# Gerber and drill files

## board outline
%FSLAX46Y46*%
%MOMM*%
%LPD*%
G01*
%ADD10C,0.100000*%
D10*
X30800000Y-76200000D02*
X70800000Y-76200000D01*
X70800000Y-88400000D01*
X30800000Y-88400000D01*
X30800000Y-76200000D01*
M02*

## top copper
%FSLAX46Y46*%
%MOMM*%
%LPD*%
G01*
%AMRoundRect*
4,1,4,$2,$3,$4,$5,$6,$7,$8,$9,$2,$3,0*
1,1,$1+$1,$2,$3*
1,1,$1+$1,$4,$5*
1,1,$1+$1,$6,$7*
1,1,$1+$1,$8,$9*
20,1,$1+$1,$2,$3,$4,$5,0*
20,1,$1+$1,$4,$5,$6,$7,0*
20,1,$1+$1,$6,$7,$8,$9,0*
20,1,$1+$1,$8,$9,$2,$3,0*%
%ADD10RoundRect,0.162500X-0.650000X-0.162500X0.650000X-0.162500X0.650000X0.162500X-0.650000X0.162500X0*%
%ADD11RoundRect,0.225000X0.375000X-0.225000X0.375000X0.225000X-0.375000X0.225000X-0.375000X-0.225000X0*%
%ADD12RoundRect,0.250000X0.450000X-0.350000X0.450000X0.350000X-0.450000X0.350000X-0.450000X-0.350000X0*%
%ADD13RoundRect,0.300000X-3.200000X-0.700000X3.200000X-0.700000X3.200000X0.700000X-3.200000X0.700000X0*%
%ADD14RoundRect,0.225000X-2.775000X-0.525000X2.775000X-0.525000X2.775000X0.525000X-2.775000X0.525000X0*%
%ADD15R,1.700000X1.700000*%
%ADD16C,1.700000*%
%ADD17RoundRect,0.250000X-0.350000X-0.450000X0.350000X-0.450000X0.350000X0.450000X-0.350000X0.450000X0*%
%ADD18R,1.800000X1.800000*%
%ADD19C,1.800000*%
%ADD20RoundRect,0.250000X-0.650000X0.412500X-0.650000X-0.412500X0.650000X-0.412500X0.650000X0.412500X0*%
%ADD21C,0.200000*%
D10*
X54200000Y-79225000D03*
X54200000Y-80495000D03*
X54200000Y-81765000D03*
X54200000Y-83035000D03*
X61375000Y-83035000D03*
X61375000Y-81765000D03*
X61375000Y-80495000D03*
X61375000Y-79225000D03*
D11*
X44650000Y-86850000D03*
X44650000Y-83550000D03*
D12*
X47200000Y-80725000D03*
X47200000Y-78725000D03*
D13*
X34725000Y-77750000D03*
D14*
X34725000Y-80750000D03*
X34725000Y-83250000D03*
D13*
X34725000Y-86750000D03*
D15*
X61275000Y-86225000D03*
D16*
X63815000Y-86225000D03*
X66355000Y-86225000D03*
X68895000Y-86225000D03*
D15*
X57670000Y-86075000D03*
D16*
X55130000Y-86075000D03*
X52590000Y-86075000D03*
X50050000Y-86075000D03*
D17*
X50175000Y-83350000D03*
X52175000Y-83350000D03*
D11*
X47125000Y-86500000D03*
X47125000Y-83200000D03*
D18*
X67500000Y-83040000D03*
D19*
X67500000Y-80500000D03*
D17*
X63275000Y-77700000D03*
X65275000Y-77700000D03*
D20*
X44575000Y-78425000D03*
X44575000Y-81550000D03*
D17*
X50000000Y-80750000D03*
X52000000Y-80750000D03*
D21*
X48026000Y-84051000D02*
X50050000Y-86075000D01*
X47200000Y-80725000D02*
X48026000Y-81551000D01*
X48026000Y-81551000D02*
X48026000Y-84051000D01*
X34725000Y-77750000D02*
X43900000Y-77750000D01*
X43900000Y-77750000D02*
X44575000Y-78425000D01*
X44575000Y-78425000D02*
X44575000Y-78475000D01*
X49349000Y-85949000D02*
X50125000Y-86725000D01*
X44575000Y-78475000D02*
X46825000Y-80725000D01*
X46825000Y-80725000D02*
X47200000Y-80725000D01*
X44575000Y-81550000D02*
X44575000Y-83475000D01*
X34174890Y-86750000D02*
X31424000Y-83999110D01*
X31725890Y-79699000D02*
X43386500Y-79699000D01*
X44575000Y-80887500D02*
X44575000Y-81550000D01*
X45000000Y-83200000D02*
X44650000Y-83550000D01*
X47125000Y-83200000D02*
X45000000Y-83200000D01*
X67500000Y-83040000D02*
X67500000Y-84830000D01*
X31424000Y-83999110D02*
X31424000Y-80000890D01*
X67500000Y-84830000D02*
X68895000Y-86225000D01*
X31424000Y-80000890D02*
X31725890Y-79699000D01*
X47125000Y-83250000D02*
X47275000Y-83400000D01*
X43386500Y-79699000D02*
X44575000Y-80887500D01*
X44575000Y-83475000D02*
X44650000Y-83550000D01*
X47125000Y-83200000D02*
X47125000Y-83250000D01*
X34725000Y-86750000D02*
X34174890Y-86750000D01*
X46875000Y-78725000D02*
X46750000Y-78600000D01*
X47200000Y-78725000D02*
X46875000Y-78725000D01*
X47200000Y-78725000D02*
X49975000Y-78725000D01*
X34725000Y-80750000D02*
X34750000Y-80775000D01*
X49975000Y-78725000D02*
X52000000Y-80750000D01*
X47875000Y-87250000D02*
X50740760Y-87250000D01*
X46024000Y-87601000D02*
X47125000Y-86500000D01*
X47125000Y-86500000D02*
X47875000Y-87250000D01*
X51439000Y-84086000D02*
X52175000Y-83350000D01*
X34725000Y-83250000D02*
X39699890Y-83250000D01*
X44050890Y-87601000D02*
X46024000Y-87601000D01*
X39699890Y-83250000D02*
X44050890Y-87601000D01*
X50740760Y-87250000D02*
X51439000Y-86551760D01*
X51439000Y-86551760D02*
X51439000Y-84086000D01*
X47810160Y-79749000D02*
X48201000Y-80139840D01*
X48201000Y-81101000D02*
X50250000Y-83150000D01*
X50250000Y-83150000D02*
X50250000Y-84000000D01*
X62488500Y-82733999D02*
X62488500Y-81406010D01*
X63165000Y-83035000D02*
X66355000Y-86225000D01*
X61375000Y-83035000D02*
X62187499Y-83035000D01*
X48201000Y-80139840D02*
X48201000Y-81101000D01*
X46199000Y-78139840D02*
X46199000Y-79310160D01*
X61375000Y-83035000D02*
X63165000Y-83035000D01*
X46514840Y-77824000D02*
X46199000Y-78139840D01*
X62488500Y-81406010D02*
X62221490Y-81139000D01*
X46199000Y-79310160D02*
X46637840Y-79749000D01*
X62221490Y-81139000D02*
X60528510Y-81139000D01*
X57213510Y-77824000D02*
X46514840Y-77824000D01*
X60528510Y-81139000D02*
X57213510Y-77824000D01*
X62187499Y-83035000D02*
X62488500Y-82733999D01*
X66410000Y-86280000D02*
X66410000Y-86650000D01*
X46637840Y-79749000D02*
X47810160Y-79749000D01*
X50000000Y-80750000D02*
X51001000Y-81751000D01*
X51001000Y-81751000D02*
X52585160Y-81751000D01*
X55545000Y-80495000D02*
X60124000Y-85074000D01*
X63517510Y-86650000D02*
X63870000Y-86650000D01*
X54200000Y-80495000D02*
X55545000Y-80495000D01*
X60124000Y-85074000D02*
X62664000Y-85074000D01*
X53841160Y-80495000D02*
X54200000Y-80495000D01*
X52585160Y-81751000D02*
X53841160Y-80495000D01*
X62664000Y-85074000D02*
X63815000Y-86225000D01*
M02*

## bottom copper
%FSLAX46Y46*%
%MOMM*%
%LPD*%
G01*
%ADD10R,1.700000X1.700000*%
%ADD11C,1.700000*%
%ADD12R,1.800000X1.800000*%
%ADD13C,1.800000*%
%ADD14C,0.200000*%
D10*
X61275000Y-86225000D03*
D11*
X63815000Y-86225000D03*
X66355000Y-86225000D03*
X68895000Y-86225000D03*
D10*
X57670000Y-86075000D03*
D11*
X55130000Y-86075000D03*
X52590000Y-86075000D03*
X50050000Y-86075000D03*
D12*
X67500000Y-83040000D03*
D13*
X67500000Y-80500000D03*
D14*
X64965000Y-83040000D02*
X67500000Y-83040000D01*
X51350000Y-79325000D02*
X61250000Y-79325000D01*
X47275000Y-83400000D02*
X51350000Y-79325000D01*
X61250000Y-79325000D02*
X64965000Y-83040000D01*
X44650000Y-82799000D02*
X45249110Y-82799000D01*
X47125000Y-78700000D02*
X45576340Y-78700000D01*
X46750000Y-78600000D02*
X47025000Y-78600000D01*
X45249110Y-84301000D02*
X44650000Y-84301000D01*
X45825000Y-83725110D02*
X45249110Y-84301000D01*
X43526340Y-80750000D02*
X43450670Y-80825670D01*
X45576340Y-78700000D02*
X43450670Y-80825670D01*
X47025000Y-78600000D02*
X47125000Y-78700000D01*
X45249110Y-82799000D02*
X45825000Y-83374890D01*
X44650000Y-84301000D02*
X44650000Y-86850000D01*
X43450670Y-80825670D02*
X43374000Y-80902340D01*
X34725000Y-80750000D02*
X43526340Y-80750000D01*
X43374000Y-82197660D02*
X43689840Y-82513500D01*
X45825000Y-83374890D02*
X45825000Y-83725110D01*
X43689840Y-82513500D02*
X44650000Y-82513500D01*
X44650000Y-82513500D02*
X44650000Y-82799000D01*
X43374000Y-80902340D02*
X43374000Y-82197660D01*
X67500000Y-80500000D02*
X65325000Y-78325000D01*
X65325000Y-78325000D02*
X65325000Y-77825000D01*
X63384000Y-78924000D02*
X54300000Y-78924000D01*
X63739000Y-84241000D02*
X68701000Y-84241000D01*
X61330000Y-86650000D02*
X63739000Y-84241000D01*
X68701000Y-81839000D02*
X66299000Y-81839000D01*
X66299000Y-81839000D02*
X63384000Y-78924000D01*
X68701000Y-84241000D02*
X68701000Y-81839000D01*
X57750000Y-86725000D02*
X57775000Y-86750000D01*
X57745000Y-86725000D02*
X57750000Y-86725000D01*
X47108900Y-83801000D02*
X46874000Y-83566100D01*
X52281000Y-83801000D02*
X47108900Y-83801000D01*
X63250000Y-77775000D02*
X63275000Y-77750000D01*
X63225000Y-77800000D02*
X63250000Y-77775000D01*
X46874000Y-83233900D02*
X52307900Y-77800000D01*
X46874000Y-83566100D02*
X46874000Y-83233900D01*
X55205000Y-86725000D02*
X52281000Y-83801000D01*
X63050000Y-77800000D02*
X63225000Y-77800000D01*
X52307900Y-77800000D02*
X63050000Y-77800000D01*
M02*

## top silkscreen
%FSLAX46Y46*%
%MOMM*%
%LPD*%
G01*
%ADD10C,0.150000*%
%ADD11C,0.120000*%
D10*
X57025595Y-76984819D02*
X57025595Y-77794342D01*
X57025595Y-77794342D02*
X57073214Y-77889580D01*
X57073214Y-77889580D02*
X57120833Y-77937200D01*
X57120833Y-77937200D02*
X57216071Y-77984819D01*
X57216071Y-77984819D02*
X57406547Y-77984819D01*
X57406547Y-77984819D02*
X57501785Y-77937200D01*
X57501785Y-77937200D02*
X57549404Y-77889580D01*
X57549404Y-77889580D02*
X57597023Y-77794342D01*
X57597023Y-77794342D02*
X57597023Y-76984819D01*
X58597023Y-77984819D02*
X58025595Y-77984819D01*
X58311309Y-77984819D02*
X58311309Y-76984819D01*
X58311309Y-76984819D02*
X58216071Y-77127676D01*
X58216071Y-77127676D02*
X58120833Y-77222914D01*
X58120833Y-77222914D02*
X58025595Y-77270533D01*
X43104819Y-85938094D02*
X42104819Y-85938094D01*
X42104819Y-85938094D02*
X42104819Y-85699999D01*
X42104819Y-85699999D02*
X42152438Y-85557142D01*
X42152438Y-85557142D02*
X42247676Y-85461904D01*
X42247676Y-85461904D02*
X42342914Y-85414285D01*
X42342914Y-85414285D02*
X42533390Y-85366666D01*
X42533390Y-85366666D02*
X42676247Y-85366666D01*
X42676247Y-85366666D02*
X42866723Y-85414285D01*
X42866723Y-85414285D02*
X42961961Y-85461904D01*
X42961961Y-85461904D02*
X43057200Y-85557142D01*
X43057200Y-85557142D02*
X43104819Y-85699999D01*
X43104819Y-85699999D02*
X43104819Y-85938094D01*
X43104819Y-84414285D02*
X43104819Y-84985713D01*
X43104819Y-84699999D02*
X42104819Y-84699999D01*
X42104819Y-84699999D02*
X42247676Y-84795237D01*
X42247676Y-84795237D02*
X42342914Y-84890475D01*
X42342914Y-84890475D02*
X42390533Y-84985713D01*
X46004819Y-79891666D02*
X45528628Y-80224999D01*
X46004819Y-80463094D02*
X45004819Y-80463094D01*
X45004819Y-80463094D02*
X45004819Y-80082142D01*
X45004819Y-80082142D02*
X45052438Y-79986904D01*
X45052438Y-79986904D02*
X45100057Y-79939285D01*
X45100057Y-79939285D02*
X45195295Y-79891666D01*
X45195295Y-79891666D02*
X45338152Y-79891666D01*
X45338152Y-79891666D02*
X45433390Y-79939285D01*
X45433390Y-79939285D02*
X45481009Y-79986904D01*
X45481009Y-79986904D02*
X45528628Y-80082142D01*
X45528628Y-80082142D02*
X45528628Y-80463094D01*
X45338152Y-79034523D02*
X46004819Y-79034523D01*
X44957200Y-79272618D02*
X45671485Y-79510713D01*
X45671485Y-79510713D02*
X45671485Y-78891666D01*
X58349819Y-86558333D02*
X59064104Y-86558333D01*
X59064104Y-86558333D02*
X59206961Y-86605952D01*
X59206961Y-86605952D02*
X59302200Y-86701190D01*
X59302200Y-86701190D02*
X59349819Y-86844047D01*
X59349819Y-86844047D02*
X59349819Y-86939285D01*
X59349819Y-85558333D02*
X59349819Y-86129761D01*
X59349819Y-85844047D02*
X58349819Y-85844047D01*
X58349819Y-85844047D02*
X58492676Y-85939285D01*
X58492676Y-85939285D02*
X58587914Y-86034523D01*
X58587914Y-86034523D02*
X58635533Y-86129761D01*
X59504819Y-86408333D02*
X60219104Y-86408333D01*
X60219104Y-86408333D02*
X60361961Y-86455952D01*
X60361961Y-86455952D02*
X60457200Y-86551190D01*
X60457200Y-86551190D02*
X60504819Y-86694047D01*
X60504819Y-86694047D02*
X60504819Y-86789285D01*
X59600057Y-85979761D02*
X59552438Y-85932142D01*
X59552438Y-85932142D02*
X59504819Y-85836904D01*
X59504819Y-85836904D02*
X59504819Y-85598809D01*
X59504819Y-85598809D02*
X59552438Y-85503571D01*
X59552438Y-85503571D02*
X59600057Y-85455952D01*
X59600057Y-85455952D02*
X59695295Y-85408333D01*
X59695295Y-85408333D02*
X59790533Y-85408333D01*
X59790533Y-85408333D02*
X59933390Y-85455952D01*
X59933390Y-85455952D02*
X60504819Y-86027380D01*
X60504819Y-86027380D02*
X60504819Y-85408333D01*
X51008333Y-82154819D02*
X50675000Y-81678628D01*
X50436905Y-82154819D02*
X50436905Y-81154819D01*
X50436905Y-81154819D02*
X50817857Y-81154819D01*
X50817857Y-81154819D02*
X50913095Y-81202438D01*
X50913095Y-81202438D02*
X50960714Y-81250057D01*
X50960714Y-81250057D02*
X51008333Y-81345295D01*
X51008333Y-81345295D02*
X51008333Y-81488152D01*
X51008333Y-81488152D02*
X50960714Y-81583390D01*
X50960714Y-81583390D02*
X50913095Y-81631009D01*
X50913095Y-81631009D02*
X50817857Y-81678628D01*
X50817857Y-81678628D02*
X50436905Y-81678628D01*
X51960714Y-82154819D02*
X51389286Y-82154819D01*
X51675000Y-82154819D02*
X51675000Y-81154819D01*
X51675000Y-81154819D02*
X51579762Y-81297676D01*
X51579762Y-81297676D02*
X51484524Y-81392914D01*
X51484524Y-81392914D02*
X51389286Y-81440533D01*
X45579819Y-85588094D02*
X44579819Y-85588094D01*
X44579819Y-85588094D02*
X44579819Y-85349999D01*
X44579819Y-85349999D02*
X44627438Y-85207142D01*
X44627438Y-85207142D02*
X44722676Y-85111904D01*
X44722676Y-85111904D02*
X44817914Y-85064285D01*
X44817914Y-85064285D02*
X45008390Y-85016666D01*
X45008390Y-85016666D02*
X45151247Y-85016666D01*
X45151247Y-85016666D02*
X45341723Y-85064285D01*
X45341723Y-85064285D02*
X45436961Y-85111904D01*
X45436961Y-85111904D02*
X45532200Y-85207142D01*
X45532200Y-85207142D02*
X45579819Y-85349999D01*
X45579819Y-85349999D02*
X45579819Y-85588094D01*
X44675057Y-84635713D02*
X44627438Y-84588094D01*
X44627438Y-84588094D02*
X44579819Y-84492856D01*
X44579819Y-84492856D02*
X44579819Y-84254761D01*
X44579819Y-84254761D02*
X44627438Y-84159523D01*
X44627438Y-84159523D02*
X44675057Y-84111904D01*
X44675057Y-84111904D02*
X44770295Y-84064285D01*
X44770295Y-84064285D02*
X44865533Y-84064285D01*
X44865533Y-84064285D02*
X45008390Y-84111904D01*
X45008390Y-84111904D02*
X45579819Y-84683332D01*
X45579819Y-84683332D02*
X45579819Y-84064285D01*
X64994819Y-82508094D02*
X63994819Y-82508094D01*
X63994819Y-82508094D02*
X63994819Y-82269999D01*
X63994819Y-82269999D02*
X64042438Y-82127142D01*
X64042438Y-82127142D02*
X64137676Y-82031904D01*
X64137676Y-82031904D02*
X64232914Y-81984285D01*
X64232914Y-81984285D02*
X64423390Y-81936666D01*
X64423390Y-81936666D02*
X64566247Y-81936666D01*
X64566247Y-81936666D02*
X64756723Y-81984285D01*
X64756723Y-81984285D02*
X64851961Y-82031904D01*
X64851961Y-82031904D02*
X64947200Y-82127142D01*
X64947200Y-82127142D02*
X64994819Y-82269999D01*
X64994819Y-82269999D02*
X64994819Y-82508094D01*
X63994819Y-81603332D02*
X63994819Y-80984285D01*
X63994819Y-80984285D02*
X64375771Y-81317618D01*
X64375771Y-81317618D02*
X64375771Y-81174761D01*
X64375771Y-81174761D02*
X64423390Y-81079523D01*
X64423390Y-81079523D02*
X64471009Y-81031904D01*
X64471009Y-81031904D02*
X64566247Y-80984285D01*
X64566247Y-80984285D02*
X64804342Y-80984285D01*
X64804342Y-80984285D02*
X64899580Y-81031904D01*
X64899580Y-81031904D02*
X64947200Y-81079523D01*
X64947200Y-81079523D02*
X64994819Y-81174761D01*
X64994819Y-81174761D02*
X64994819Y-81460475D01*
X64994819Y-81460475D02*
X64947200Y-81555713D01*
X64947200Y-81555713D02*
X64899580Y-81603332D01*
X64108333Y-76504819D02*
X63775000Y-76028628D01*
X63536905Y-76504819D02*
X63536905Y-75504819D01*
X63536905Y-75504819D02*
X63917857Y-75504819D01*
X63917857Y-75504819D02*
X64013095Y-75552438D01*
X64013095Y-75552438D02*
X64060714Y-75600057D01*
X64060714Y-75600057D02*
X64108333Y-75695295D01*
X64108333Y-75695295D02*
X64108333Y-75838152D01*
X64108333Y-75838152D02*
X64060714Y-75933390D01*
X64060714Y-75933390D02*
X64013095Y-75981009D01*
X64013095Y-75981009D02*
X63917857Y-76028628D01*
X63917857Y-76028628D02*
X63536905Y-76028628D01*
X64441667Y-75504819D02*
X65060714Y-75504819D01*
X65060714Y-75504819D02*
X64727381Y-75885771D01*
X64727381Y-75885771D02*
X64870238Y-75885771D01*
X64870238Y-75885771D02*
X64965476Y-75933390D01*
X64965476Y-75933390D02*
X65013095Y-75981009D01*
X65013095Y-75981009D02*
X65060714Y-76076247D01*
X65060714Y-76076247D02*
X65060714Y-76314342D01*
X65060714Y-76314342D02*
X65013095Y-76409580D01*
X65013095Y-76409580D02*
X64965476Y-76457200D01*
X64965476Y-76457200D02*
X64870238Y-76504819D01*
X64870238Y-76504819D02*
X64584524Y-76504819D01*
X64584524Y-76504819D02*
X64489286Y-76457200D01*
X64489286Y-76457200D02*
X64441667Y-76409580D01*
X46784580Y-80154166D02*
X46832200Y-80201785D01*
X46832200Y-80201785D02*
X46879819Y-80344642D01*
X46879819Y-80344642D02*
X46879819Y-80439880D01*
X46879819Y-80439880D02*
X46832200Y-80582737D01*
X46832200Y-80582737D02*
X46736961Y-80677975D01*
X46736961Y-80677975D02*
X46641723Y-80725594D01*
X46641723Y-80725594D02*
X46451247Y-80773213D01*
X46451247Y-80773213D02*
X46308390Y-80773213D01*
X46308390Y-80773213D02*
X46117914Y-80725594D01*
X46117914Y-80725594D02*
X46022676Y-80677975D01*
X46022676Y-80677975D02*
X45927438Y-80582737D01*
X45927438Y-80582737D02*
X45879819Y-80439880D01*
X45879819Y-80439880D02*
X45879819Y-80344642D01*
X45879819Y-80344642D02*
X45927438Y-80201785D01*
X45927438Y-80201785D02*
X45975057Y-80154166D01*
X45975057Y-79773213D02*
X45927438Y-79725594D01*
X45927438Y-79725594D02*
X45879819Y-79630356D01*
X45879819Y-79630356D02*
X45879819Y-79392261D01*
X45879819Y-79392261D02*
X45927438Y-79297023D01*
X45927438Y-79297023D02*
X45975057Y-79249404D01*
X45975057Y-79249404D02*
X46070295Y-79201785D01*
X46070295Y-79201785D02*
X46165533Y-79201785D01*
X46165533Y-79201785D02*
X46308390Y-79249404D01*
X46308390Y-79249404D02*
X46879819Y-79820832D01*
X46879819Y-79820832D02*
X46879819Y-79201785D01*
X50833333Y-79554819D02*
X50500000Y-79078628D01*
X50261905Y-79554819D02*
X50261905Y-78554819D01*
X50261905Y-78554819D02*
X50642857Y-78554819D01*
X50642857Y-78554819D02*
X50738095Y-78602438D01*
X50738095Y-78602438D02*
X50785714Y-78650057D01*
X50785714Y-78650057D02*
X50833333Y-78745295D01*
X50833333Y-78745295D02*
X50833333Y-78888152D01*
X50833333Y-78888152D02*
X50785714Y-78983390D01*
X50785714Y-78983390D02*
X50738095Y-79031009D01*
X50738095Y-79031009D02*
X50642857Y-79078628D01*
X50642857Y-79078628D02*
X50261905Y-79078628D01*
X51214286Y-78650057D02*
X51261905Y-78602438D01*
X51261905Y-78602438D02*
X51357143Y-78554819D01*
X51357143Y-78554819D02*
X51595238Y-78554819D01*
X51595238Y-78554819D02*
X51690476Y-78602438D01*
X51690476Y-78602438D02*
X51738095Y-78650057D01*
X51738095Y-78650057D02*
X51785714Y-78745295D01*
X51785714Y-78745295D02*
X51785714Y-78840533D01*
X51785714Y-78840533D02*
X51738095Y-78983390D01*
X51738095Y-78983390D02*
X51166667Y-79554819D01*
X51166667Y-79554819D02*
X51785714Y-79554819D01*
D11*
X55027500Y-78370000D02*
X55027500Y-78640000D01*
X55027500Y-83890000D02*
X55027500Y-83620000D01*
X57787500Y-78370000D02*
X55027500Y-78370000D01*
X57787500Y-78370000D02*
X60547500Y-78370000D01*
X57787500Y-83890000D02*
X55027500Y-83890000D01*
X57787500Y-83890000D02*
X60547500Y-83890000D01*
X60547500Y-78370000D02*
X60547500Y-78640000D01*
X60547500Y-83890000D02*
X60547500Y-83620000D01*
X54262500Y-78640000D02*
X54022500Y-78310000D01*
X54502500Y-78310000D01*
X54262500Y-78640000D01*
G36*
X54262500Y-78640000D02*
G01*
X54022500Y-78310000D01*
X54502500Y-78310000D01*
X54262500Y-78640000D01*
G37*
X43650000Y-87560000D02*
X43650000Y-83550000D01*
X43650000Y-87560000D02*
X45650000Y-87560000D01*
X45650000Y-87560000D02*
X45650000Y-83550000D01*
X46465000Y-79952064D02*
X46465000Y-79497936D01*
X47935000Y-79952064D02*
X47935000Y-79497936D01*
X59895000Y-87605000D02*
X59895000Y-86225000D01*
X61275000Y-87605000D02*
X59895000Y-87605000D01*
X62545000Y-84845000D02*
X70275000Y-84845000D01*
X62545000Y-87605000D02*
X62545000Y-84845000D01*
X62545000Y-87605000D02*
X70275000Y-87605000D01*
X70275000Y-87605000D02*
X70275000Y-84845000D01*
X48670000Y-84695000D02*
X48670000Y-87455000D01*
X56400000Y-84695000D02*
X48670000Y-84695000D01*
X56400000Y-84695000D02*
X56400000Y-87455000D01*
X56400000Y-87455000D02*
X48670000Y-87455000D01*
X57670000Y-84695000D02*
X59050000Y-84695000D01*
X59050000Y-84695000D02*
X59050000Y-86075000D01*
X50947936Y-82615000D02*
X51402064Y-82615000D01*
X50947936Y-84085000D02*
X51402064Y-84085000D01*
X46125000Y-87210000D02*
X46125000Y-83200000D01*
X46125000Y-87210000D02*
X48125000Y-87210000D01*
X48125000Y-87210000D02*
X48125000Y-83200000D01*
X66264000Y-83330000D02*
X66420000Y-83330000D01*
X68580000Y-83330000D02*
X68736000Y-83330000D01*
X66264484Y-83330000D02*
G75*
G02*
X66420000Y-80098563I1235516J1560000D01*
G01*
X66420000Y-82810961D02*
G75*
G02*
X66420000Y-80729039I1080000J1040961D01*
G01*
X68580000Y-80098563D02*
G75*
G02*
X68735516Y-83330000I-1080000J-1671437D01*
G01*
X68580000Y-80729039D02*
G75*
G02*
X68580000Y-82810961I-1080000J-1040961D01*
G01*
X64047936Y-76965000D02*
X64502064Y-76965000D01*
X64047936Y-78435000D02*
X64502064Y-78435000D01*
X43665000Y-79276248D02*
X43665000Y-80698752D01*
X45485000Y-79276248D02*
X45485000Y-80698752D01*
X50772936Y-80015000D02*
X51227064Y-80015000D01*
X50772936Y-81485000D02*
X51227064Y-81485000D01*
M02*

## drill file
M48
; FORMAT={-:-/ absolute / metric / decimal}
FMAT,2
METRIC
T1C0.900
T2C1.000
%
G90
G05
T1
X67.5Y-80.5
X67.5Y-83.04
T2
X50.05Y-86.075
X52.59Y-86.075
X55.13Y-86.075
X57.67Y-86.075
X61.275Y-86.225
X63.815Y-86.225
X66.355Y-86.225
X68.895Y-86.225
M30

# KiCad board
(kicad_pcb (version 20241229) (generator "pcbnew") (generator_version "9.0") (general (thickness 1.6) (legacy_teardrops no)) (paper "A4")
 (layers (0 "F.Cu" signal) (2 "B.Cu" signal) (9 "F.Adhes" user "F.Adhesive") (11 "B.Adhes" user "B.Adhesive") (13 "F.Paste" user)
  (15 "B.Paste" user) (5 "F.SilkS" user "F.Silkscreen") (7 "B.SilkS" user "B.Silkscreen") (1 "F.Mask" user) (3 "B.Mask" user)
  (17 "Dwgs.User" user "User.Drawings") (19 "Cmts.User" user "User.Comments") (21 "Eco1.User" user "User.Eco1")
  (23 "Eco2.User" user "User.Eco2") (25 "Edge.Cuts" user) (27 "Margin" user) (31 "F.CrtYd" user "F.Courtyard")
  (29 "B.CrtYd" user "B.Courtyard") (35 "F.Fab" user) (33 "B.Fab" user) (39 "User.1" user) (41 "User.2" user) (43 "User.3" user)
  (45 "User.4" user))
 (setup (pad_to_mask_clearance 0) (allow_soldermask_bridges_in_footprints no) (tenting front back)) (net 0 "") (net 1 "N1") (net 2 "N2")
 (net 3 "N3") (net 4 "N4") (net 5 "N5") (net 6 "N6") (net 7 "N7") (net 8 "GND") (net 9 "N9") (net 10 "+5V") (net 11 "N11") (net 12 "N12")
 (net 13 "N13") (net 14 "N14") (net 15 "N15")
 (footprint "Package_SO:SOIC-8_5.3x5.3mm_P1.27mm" (layer "F.Cu") (at 57.7875 81.13)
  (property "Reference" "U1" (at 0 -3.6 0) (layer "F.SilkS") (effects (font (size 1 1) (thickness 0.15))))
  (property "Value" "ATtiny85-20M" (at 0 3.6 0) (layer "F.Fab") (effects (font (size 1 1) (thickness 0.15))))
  (fp_line (start -2.76 -2.76) (end -2.76 -2.49) (stroke (width 0.12) (type solid)) (layer "F.SilkS"))
  (fp_line (start -2.76 2.76) (end -2.76 2.49) (stroke (width 0.12) (type solid)) (layer "F.SilkS"))
  (fp_line (start 0 -2.76) (end -2.76 -2.76) (stroke (width 0.12) (type solid)) (layer "F.SilkS"))
  (fp_line (start 0 -2.76) (end 2.76 -2.76) (stroke (width 0.12) (type solid)) (layer "F.SilkS"))
  (fp_line (start 0 2.76) (end -2.76 2.76) (stroke (width 0.12) (type solid)) (layer "F.SilkS"))
  (fp_line (start 0 2.76) (end 2.76 2.76) (stroke (width 0.12) (type solid)) (layer "F.SilkS"))
  (fp_line (start 2.76 -2.76) (end 2.76 -2.49) (stroke (width 0.12) (type solid)) (layer "F.SilkS"))
  (fp_line (start 2.76 2.76) (end 2.76 2.49) (stroke (width 0.12) (type solid)) (layer "F.SilkS"))
  (fp_poly (pts (xy -3.525 -2.49) (xy -3.765 -2.82) (xy -3.285 -2.82)) (stroke (width 0.12) (type solid)) (fill yes) (layer "F.SilkS"))
  (pad "1" smd roundrect (at -3.5875 -1.905) (size 1.625 0.65) (layers "F.Cu" "F.Mask" "F.Paste") (roundrect_rratio 0.25) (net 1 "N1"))
  (pad "2" smd roundrect (at -3.5875 -0.635) (size 1.625 0.65) (layers "F.Cu" "F.Mask" "F.Paste") (roundrect_rratio 0.25) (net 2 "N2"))
  (pad "3" smd roundrect (at -3.5875 0.635) (size 1.625 0.65) (layers "F.Cu" "F.Mask" "F.Paste") (roundrect_rratio 0.25) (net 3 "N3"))
  (pad "4" smd roundrect (at -3.5875 1.905) (size 1.625 0.65) (layers "F.Cu" "F.Mask" "F.Paste") (roundrect_rratio 0.25) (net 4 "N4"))
  (pad "5" smd roundrect (at 3.5875 1.905) (size 1.625 0.65) (layers "F.Cu" "F.Mask" "F.Paste") (roundrect_rratio 0.25) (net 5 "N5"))
  (pad "6" smd roundrect (at 3.5875 0.635) (size 1.625 0.65) (layers "F.Cu" "F.Mask" "F.Paste") (roundrect_rratio 0.25) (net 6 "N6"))
  (pad "7" smd roundrect (at 3.5875 -0.635) (size 1.625 0.65) (layers "F.Cu" "F.Mask" "F.Paste") (roundrect_rratio 0.25) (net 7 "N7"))
  (pad "8" smd roundrect (at 3.5875 -1.905) (size 1.625 0.65) (layers "F.Cu" "F.Mask" "F.Paste") (roundrect_rratio 0.25) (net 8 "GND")))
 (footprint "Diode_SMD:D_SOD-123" (layer "F.Cu") (at 44.65 85.2 90)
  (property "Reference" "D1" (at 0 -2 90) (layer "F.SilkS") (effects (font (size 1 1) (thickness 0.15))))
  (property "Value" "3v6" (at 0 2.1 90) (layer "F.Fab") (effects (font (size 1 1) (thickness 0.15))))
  (fp_line (start -2.36 -1) (end 1.65 -1) (stroke (width 0.12) (type solid)) (layer "F.SilkS"))
  (fp_line (start -2.36 -1) (end -2.36 1) (stroke (width 0.12) (type solid)) (layer "F.SilkS"))
  (fp_line (start -2.36 1) (end 1.65 1) (stroke (width 0.12) (type solid)) (layer "F.SilkS"))
  (pad "1" smd roundrect (at -1.65 0 90) (size 0.9 1.2) (layers "F.Cu" "F.Mask" "F.Paste") (roundrect_rratio 0.25) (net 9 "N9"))
  (pad "2" smd roundrect (at 1.65 0 90) (size 0.9 1.2) (layers "F.Cu" "F.Mask" "F.Paste") (roundrect_rratio 0.25) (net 8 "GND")))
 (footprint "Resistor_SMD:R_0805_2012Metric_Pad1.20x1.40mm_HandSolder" (layer "F.Cu") (at 47.2 79.725 90)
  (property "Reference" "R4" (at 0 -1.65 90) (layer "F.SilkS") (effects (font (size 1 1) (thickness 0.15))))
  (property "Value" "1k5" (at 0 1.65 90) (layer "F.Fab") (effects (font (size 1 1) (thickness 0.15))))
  (fp_line (start -0.227064 -0.735) (end 0.227064 -0.735) (stroke (width 0.12) (type solid)) (layer "F.SilkS"))
  (fp_line (start -0.227064 0.735) (end 0.227064 0.735) (stroke (width 0.12) (type solid)) (layer "F.SilkS"))
  (pad "1" smd roundrect (at -1 0 90) (size 1.2 1.4) (layers "F.Cu" "F.Mask" "F.Paste") (roundrect_rratio 0.208333) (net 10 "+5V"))
  (pad "2" smd roundrect (at 1 0 90) (size 1.2 1.4) (layers "F.Cu" "F.Mask" "F.Paste") (roundrect_rratio 0.208333) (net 9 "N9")))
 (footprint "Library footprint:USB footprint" (layer "F.Cu") (at 34.725 86.75)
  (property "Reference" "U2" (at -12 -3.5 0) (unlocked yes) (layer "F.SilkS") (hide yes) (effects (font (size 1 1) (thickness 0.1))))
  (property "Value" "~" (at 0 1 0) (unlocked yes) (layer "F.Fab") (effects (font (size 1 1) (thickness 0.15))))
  (pad "1" smd roundrect (at 0 -9) (size 7 2) (layers "F.Cu" "F.Mask" "F.Paste") (roundrect_rratio 0.15) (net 10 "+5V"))
  (pad "2" smd roundrect (at 0 -6) (size 6 1.5) (layers "F.Cu" "F.Mask" "F.Paste") (roundrect_rratio 0.15) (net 9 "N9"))
  (pad "3" smd roundrect (at 0 -3.5) (size 6 1.5) (layers "F.Cu" "F.Mask" "F.Paste") (roundrect_rratio 0.15) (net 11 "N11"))
  (pad "4" smd roundrect (at 0 0) (size 7 2) (layers "F.Cu" "F.Mask" "F.Paste") (roundrect_rratio 0.15) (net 8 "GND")))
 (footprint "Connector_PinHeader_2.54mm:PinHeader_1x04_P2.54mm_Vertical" (layer "F.Cu") (at 61.275 86.225 90)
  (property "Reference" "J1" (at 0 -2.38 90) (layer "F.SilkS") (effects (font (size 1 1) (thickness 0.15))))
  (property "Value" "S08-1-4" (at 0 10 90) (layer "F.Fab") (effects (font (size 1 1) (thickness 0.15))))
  (fp_line (start -1.38 -1.38) (end 0 -1.38) (stroke (width 0.12) (type solid)) (layer "F.SilkS"))
  (fp_line (start -1.38 0) (end -1.38 -1.38) (stroke (width 0.12) (type solid)) (layer "F.SilkS"))
  (fp_line (start 1.38 1.27) (end 1.38 9) (stroke (width 0.12) (type solid)) (layer "F.SilkS"))
  (fp_line (start -1.38 1.27) (end 1.38 1.27) (stroke (width 0.12) (type solid)) (layer "F.SilkS"))
  (fp_line (start -1.38 1.27) (end -1.38 9) (stroke (width 0.12) (type solid)) (layer "F.SilkS"))
  (fp_line (start -1.38 9) (end 1.38 9) (stroke (width 0.12) (type solid)) (layer "F.SilkS"))
  (pad "1" thru_hole rect (at 0 0 90) (size 1.7 1.7) (drill 1) (layers "*.Cu" "*.Mask") (remove_unused_layers no) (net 1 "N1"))
  (pad "2" thru_hole circle (at 0 2.54 90) (size 1.7 1.7) (drill 1) (layers "*.Cu" "*.Mask") (remove_unused_layers no) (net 2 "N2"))
  (pad "3" thru_hole circle (at 0 5.08 90) (size 1.7 1.7) (drill 1) (layers "*.Cu" "*.Mask") (remove_unused_layers no) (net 5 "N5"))
  (pad "4" thru_hole circle (at 0 7.62 90) (size 1.7 1.7) (drill 1) (layers "*.Cu" "*.Mask") (remove_unused_layers no) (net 8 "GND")))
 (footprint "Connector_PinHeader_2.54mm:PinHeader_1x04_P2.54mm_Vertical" (layer "F.Cu") (at 57.67 86.075 -90)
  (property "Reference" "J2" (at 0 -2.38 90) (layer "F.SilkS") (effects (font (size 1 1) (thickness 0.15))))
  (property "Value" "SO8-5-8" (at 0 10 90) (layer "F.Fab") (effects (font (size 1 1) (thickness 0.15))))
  (fp_line (start -1.38 9) (end 1.38 9) (stroke (width 0.12) (type solid)) (layer "F.SilkS"))
  (fp_line (start -1.38 1.27) (end -1.38 9) (stroke (width 0.12) (type solid)) (layer "F.SilkS"))
  (fp_line (start -1.38 1.27) (end 1.38 1.27) (stroke (width 0.12) (type solid)) (layer "F.SilkS"))
  (fp_line (start 1.38 1.27) (end 1.38 9) (stroke (width 0.12) (type solid)) (layer "F.SilkS"))
  (fp_line (start -1.38 0) (end -1.38 -1.38) (stroke (width 0.12) (type solid)) (layer "F.SilkS"))
  (fp_line (start -1.38 -1.38) (end 0 -1.38) (stroke (width 0.12) (type solid)) (layer "F.SilkS"))
  (pad "1" thru_hole rect (at 0 0 270) (size 1.7 1.7) (drill 1) (layers "*.Cu" "*.Mask") (remove_unused_layers no) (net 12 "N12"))
  (pad "2" thru_hole circle (at 0 2.54 270) (size 1.7 1.7) (drill 1) (layers "*.Cu" "*.Mask") (remove_unused_layers no) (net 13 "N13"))
  (pad "3" thru_hole circle (at 0 5.08 270) (size 1.7 1.7) (drill 1) (layers "*.Cu" "*.Mask") (remove_unused_layers no) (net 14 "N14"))
  (pad "4" thru_hole circle (at 0 7.62 270) (size 1.7 1.7) (drill 1) (layers "*.Cu" "*.Mask") (remove_unused_layers no) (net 10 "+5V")))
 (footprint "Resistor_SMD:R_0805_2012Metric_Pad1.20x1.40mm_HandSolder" (layer "F.Cu") (at 51.175 83.35)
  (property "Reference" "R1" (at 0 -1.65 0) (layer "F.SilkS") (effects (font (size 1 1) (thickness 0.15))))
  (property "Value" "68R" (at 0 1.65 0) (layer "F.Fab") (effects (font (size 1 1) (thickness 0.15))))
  (fp_line (start -0.227064 -0.735) (end 0.227064 -0.735) (stroke (width 0.12) (type solid)) (layer "F.SilkS"))
  (fp_line (start -0.227064 0.735) (end 0.227064 0.735) (stroke (width 0.12) (type solid)) (layer "F.SilkS"))
  (pad "1" smd roundrect (at -1 0) (size 1.2 1.4) (layers "F.Cu" "F.Mask" "F.Paste") (roundrect_rratio 0.208333) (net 5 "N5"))
  (pad "2" smd roundrect (at 1 0) (size 1.2 1.4) (layers "F.Cu" "F.Mask" "F.Paste") (roundrect_rratio 0.208333) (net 11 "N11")))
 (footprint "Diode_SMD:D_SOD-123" (layer "F.Cu") (at 47.125 84.85 90)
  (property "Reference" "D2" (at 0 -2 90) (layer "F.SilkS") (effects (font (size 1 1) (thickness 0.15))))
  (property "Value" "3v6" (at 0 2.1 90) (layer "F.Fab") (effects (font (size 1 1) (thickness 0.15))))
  (fp_line (start -2.36 -1) (end 1.65 -1) (stroke (width 0.12) (type solid)) (layer "F.SilkS"))
  (fp_line (start -2.36 -1) (end -2.36 1) (stroke (width 0.12) (type solid)) (layer "F.SilkS"))
  (fp_line (start -2.36 1) (end 1.65 1) (stroke (width 0.12) (type solid)) (layer "F.SilkS"))
  (pad "1" smd roundrect (at -1.65 0 90) (size 0.9 1.2) (layers "F.Cu" "F.Mask" "F.Paste") (roundrect_rratio 0.25) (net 11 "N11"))
  (pad "2" smd roundrect (at 1.65 0 90) (size 0.9 1.2) (layers "F.Cu" "F.Mask" "F.Paste") (roundrect_rratio 0.25) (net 8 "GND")))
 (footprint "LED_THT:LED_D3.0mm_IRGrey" (layer "F.Cu") (at 67.5 83.04 90)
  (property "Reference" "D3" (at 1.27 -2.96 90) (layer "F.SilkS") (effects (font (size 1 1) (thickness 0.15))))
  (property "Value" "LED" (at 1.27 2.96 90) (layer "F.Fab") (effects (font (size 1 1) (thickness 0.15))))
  (fp_line (start -0.29 -1.236) (end -0.29 -1.08) (stroke (width 0.12) (type solid)) (layer "F.SilkS"))
  (fp_line (start -0.29 1.08) (end -0.29 1.236) (stroke (width 0.12) (type solid)) (layer "F.SilkS"))
  (fp_arc (start -0.29 -1.235516) (mid 1.36566 -1.987699) (end 2.941437 -1.08) (stroke (width 0.12) (type solid)) (layer "F.SilkS"))
  (fp_arc (start 0.229039 -1.08) (mid 1.27 -1.5) (end 2.310961 -1.08) (stroke (width 0.12) (type solid)) (layer "F.SilkS"))
  (fp_arc (start 2.941437 1.08) (mid 1.36566 1.987699) (end -0.29 1.235516) (stroke (width 0.12) (type solid)) (layer "F.SilkS"))
  (fp_arc (start 2.310961 1.08) (mid 1.27 1.5) (end 0.229039 1.08) (stroke (width 0.12) (type solid)) (layer "F.SilkS"))
  (pad "1" thru_hole rect (at 0 0 90) (size 1.8 1.8) (drill 0.9) (layers "*.Cu" "*.Mask") (remove_unused_layers no) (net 8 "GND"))
  (pad "2" thru_hole circle (at 2.54 0 90) (size 1.8 1.8) (drill 0.9) (layers "*.Cu" "*.Mask") (remove_unused_layers no) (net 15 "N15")))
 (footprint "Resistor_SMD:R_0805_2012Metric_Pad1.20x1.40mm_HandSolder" (layer "F.Cu") (at 64.275 77.7)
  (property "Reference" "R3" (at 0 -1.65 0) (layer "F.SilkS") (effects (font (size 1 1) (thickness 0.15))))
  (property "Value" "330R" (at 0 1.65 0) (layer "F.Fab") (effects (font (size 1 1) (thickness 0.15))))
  (fp_line (start -0.227064 -0.735) (end 0.227064 -0.735) (stroke (width 0.12) (type solid)) (layer "F.SilkS"))
  (fp_line (start -0.227064 0.735) (end 0.227064 0.735) (stroke (width 0.12) (type solid)) (layer "F.SilkS"))
  (pad "1" smd roundrect (at -1 0) (size 1.2 1.4) (layers "F.Cu" "F.Mask" "F.Paste") (roundrect_rratio 0.208333) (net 13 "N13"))
  (pad "2" smd roundrect (at 1 0) (size 1.2 1.4) (layers "F.Cu" "F.Mask" "F.Paste") (roundrect_rratio 0.208333) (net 15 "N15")))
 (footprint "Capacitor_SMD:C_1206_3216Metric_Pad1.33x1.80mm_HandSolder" (layer "F.Cu") (at 44.575 79.9875 -90)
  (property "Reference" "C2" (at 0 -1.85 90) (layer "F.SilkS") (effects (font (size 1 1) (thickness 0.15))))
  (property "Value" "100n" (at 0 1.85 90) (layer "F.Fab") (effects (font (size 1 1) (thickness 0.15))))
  (fp_line (start -0.711252 0.91) (end 0.711252 0.91) (stroke (width 0.12) (type solid)) (layer "F.SilkS"))
  (fp_line (start -0.711252 -0.91) (end 0.711252 -0.91) (stroke (width 0.12) (type solid)) (layer "F.SilkS"))
  (pad "1" smd roundrect (at -1.5625 0 270) (size 1.325 1.8) (layers "F.Cu" "F.Mask" "F.Paste") (roundrect_rratio 0.188679) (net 10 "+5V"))
  (pad "2" smd roundrect (at 1.5625 0 270) (size 1.325 1.8) (layers "F.Cu" "F.Mask" "F.Paste") (roundrect_rratio 0.188679) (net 8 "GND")))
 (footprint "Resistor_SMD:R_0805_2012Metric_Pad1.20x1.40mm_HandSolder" (layer "F.Cu") (at 51 80.75)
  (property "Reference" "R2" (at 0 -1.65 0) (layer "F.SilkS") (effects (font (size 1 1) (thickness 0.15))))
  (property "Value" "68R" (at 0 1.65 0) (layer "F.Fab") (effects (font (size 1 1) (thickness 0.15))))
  (fp_line (start -0.227064 -0.735) (end 0.227064 -0.735) (stroke (width 0.12) (type solid)) (layer "F.SilkS"))
  (fp_line (start -0.227064 0.735) (end 0.227064 0.735) (stroke (width 0.12) (type solid)) (layer "F.SilkS"))
  (pad "1" smd roundrect (at -1 0) (size 1.2 1.4) (layers "F.Cu" "F.Mask" "F.Paste") (roundrect_rratio 0.208333) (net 2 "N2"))
  (pad "2" smd roundrect (at 1 0) (size 1.2 1.4) (layers "F.Cu" "F.Mask" "F.Paste") (roundrect_rratio 0.208333) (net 9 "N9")))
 (gr_rect (start 30.8 76.2) (end 70.8 88.4) (stroke (width 0.1) (type solid)) (fill no) (layer "Edge.Cuts"))
 (segment (start 48.026 84.051) (end 50.05 86.075) (width 0.2) (layer "F.Cu") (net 10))
 (segment (start 47.2 80.725) (end 48.026 81.551) (width 0.2) (layer "F.Cu") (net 10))
 (segment (start 48.026 81.551) (end 48.026 84.051) (width 0.2) (layer "F.Cu") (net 10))
 (segment (start 34.725 77.75) (end 43.9 77.75) (width 0.2) (layer "F.Cu") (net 10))
 (segment (start 43.9 77.75) (end 44.575 78.425) (width 0.2) (layer "F.Cu") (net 10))
 (segment (start 44.575 78.425) (end 44.575 78.475) (width 0.2) (layer "F.Cu") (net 10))
 (segment (start 49.349 85.949) (end 50.125 86.725) (width 0.2) (layer "F.Cu") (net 10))
 (segment (start 44.575 78.475) (end 46.825 80.725) (width 0.2) (layer "F.Cu") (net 10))
 (segment (start 46.825 80.725) (end 47.2 80.725) (width 0.2) (layer "F.Cu") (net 10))
 (segment (start 44.575 81.55) (end 44.575 83.475) (width 0.2) (layer "F.Cu") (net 8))
 (segment (start 34.17489 86.75) (end 31.424 83.99911) (width 0.2) (layer "F.Cu") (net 8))
 (segment (start 31.72589 79.699) (end 43.3865 79.699) (width 0.2) (layer "F.Cu") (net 8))
 (segment (start 44.575 80.8875) (end 44.575 81.55) (width 0.2) (layer "F.Cu") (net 8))
 (segment (start 45 83.2) (end 44.65 83.55) (width 0.2) (layer "F.Cu") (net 8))
 (segment (start 47.125 83.2) (end 45 83.2) (width 0.2) (layer "F.Cu") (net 8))
 (segment (start 67.5 83.04) (end 67.5 84.83) (width 0.2) (layer "F.Cu") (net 8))
 (segment (start 31.424 83.99911) (end 31.424 80.00089) (width 0.2) (layer "F.Cu") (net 8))
 (segment (start 67.5 84.83) (end 68.895 86.225) (width 0.2) (layer "F.Cu") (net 8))
 (segment (start 31.424 80.00089) (end 31.72589 79.699) (width 0.2) (layer "F.Cu") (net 8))
 (segment (start 47.125 83.25) (end 47.275 83.4) (width 0.2) (layer "F.Cu") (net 8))
 (segment (start 43.3865 79.699) (end 44.575 80.8875) (width 0.2) (layer "F.Cu") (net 8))
 (segment (start 44.575 83.475) (end 44.65 83.55) (width 0.2) (layer "F.Cu") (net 8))
 (segment (start 47.125 83.2) (end 47.125 83.25) (width 0.2) (layer "F.Cu") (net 8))
 (segment (start 34.725 86.75) (end 34.17489 86.75) (width 0.2) (layer "F.Cu") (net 8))
 (segment (start 64.965 83.04) (end 67.5 83.04) (width 0.2) (layer "B.Cu") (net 8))
 (segment (start 51.35 79.325) (end 61.25 79.325) (width 0.2) (layer "B.Cu") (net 8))
 (segment (start 47.275 83.4) (end 51.35 79.325) (width 0.2) (layer "B.Cu") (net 8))
 (segment (start 61.25 79.325) (end 64.965 83.04) (width 0.2) (layer "B.Cu") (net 8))
 (segment (start 46.875 78.725) (end 46.75 78.6) (width 0.2) (layer "F.Cu") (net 9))
 (segment (start 47.2 78.725) (end 46.875 78.725) (width 0.2) (layer "F.Cu") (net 9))
 (segment (start 47.2 78.725) (end 49.975 78.725) (width 0.2) (layer "F.Cu") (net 9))
 (segment (start 34.725 80.75) (end 34.75 80.775) (width 0.2) (layer "F.Cu") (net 9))
 (segment (start 49.975 78.725) (end 52 80.75) (width 0.2) (layer "F.Cu") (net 9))
 (segment (start 44.65 82.799) (end 45.24911 82.799) (width 0.2) (layer "B.Cu") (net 9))
 (segment (start 47.125 78.7) (end 45.57634 78.7) (width 0.2) (layer "B.Cu") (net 9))
 (segment (start 46.75 78.6) (end 47.025 78.6) (width 0.2) (layer "B.Cu") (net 9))
 (segment (start 45.24911 84.301) (end 44.65 84.301) (width 0.2) (layer "B.Cu") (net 9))
 (segment (start 45.825 83.72511) (end 45.24911 84.301) (width 0.2) (layer "B.Cu") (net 9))
 (segment (start 43.52634 80.75) (end 43.45067 80.82567) (width 0.2) (layer "B.Cu") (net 9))
 (segment (start 45.57634 78.7) (end 43.45067 80.82567) (width 0.2) (layer "B.Cu") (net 9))
 (segment (start 47.025 78.6) (end 47.125 78.7) (width 0.2) (layer "B.Cu") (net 9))
 (segment (start 45.24911 82.799) (end 45.825 83.37489) (width 0.2) (layer "B.Cu") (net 9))
 (segment (start 44.65 84.301) (end 44.65 86.85) (width 0.2) (layer "B.Cu") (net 9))
 (segment (start 43.45067 80.82567) (end 43.374 80.90234) (width 0.2) (layer "B.Cu") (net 9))
 (segment (start 34.725 80.75) (end 43.52634 80.75) (width 0.2) (layer "B.Cu") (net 9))
 (segment (start 43.374 82.19766) (end 43.68984 82.5135) (width 0.2) (layer "B.Cu") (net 9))
 (segment (start 45.825 83.37489) (end 45.825 83.72511) (width 0.2) (layer "B.Cu") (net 9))
 (segment (start 43.68984 82.5135) (end 44.65 82.5135) (width 0.2) (layer "B.Cu") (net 9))
 (segment (start 44.65 82.5135) (end 44.65 82.799) (width 0.2) (layer "B.Cu") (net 9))
 (segment (start 43.374 80.90234) (end 43.374 82.19766) (width 0.2) (layer "B.Cu") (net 9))
 (segment (start 47.875 87.25) (end 50.74076 87.25) (width 0.2) (layer "F.Cu") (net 11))
 (segment (start 46.024 87.601) (end 47.125 86.5) (width 0.2) (layer "F.Cu") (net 11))
 (segment (start 47.125 86.5) (end 47.875 87.25) (width 0.2) (layer "F.Cu") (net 11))
 (segment (start 51.439 84.086) (end 52.175 83.35) (width 0.2) (layer "F.Cu") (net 11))
 (segment (start 34.725 83.25) (end 39.69989 83.25) (width 0.2) (layer "F.Cu") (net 11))
 (segment (start 44.05089 87.601) (end 46.024 87.601) (width 0.2) (layer "F.Cu") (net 11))
 (segment (start 39.69989 83.25) (end 44.05089 87.601) (width 0.2) (layer "F.Cu") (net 11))
 (segment (start 50.74076 87.25) (end 51.439 86.55176) (width 0.2) (layer "F.Cu") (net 11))
 (segment (start 51.439 86.55176) (end 51.439 84.086) (width 0.2) (layer "F.Cu") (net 11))
 (segment (start 67.5 80.5) (end 65.325 78.325) (width 0.2) (layer "B.Cu") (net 15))
 (segment (start 65.325 78.325) (end 65.325 77.825) (width 0.2) (layer "B.Cu") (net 15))
 (segment (start 63.384 78.924) (end 54.3 78.924) (width 0.2) (layer "B.Cu") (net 1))
 (segment (start 63.739 84.241) (end 68.701 84.241) (width 0.2) (layer "B.Cu") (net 1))
 (segment (start 61.33 86.65) (end 63.739 84.241) (width 0.2) (layer "B.Cu") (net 1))
 (segment (start 68.701 81.839) (end 66.299 81.839) (width 0.2) (layer "B.Cu") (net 1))
 (segment (start 66.299 81.839) (end 63.384 78.924) (width 0.2) (layer "B.Cu") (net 1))
 (segment (start 68.701 84.241) (end 68.701 81.839) (width 0.2) (layer "B.Cu") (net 1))
 (segment (start 47.81016 79.749) (end 48.201 80.13984) (width 0.2) (layer "F.Cu") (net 5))
 (segment (start 48.201 81.101) (end 50.25 83.15) (width 0.2) (layer "F.Cu") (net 5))
 (segment (start 50.25 83.15) (end 50.25 84) (width 0.2) (layer "F.Cu") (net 5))
 (segment (start 62.4885 82.733999) (end 62.4885 81.40601) (width 0.2) (layer "F.Cu") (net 5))
 (segment (start 63.165 83.035) (end 66.355 86.225) (width 0.2) (layer "F.Cu") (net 5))
 (segment (start 61.375 83.035) (end 62.187499 83.035) (width 0.2) (layer "F.Cu") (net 5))
 (segment (start 48.201 80.13984) (end 48.201 81.101) (width 0.2) (layer "F.Cu") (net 5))
 (segment (start 46.199 78.13984) (end 46.199 79.31016) (width 0.2) (layer "F.Cu") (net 5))
 (segment (start 61.375 83.035) (end 63.165 83.035) (width 0.2) (layer "F.Cu") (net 5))
 (segment (start 46.51484 77.824) (end 46.199 78.13984) (width 0.2) (layer "F.Cu") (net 5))
 (segment (start 62.4885 81.40601) (end 62.22149 81.139) (width 0.2) (layer "F.Cu") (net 5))
 (segment (start 46.199 79.31016) (end 46.63784 79.749) (width 0.2) (layer "F.Cu") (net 5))
 (segment (start 62.22149 81.139) (end 60.52851 81.139) (width 0.2) (layer "F.Cu") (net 5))
 (segment (start 57.21351 77.824) (end 46.51484 77.824) (width 0.2) (layer "F.Cu") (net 5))
 (segment (start 60.52851 81.139) (end 57.21351 77.824) (width 0.2) (layer "F.Cu") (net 5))
 (segment (start 62.187499 83.035) (end 62.4885 82.733999) (width 0.2) (layer "F.Cu") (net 5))
 (segment (start 66.41 86.28) (end 66.41 86.65) (width 0.2) (layer "F.Cu") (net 5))
 (segment (start 46.63784 79.749) (end 47.81016 79.749) (width 0.2) (layer "F.Cu") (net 5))
 (segment (start 50 80.75) (end 51.001 81.751) (width 0.2) (layer "F.Cu") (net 2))
 (segment (start 51.001 81.751) (end 52.58516 81.751) (width 0.2) (layer "F.Cu") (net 2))
 (segment (start 55.545 80.495) (end 60.124 85.074) (width 0.2) (layer "F.Cu") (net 2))
 (segment (start 63.51751 86.65) (end 63.87 86.65) (width 0.2) (layer "F.Cu") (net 2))
 (segment (start 54.2 80.495) (end 55.545 80.495) (width 0.2) (layer "F.Cu") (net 2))
 (segment (start 60.124 85.074) (end 62.664 85.074) (width 0.2) (layer "F.Cu") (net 2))
 (segment (start 53.84116 80.495) (end 54.2 80.495) (width 0.2) (layer "F.Cu") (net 2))
 (segment (start 52.58516 81.751) (end 53.84116 80.495) (width 0.2) (layer "F.Cu") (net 2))
 (segment (start 62.664 85.074) (end 63.815 86.225) (width 0.2) (layer "F.Cu") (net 2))
 (segment (start 57.75 86.725) (end 57.775 86.75) (width 0.2) (layer "B.Cu") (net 12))
 (segment (start 57.745 86.725) (end 57.75 86.725) (width 0.2) (layer "B.Cu") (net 12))
 (segment (start 47.1089 83.801) (end 46.874 83.5661) (width 0.2) (layer "B.Cu") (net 13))
 (segment (start 52.281 83.801) (end 47.1089 83.801) (width 0.2) (layer "B.Cu") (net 13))
 (segment (start 63.25 77.775) (end 63.275 77.75) (width 0.2) (layer "B.Cu") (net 13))
 (segment (start 63.225 77.8) (end 63.25 77.775) (width 0.2) (layer "B.Cu") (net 13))
 (segment (start 46.874 83.2339) (end 52.3079 77.8) (width 0.2) (layer "B.Cu") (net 13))
 (segment (start 46.874 83.5661) (end 46.874 83.2339) (width 0.2) (layer "B.Cu") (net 13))
 (segment (start 55.205 86.725) (end 52.281 83.801) (width 0.2) (layer "B.Cu") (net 13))
 (segment (start 63.05 77.8) (end 63.225 77.8) (width 0.2) (layer "B.Cu") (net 13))
 (segment (start 52.3079 77.8) (end 63.05 77.8) (width 0.2) (layer "B.Cu") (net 13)))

